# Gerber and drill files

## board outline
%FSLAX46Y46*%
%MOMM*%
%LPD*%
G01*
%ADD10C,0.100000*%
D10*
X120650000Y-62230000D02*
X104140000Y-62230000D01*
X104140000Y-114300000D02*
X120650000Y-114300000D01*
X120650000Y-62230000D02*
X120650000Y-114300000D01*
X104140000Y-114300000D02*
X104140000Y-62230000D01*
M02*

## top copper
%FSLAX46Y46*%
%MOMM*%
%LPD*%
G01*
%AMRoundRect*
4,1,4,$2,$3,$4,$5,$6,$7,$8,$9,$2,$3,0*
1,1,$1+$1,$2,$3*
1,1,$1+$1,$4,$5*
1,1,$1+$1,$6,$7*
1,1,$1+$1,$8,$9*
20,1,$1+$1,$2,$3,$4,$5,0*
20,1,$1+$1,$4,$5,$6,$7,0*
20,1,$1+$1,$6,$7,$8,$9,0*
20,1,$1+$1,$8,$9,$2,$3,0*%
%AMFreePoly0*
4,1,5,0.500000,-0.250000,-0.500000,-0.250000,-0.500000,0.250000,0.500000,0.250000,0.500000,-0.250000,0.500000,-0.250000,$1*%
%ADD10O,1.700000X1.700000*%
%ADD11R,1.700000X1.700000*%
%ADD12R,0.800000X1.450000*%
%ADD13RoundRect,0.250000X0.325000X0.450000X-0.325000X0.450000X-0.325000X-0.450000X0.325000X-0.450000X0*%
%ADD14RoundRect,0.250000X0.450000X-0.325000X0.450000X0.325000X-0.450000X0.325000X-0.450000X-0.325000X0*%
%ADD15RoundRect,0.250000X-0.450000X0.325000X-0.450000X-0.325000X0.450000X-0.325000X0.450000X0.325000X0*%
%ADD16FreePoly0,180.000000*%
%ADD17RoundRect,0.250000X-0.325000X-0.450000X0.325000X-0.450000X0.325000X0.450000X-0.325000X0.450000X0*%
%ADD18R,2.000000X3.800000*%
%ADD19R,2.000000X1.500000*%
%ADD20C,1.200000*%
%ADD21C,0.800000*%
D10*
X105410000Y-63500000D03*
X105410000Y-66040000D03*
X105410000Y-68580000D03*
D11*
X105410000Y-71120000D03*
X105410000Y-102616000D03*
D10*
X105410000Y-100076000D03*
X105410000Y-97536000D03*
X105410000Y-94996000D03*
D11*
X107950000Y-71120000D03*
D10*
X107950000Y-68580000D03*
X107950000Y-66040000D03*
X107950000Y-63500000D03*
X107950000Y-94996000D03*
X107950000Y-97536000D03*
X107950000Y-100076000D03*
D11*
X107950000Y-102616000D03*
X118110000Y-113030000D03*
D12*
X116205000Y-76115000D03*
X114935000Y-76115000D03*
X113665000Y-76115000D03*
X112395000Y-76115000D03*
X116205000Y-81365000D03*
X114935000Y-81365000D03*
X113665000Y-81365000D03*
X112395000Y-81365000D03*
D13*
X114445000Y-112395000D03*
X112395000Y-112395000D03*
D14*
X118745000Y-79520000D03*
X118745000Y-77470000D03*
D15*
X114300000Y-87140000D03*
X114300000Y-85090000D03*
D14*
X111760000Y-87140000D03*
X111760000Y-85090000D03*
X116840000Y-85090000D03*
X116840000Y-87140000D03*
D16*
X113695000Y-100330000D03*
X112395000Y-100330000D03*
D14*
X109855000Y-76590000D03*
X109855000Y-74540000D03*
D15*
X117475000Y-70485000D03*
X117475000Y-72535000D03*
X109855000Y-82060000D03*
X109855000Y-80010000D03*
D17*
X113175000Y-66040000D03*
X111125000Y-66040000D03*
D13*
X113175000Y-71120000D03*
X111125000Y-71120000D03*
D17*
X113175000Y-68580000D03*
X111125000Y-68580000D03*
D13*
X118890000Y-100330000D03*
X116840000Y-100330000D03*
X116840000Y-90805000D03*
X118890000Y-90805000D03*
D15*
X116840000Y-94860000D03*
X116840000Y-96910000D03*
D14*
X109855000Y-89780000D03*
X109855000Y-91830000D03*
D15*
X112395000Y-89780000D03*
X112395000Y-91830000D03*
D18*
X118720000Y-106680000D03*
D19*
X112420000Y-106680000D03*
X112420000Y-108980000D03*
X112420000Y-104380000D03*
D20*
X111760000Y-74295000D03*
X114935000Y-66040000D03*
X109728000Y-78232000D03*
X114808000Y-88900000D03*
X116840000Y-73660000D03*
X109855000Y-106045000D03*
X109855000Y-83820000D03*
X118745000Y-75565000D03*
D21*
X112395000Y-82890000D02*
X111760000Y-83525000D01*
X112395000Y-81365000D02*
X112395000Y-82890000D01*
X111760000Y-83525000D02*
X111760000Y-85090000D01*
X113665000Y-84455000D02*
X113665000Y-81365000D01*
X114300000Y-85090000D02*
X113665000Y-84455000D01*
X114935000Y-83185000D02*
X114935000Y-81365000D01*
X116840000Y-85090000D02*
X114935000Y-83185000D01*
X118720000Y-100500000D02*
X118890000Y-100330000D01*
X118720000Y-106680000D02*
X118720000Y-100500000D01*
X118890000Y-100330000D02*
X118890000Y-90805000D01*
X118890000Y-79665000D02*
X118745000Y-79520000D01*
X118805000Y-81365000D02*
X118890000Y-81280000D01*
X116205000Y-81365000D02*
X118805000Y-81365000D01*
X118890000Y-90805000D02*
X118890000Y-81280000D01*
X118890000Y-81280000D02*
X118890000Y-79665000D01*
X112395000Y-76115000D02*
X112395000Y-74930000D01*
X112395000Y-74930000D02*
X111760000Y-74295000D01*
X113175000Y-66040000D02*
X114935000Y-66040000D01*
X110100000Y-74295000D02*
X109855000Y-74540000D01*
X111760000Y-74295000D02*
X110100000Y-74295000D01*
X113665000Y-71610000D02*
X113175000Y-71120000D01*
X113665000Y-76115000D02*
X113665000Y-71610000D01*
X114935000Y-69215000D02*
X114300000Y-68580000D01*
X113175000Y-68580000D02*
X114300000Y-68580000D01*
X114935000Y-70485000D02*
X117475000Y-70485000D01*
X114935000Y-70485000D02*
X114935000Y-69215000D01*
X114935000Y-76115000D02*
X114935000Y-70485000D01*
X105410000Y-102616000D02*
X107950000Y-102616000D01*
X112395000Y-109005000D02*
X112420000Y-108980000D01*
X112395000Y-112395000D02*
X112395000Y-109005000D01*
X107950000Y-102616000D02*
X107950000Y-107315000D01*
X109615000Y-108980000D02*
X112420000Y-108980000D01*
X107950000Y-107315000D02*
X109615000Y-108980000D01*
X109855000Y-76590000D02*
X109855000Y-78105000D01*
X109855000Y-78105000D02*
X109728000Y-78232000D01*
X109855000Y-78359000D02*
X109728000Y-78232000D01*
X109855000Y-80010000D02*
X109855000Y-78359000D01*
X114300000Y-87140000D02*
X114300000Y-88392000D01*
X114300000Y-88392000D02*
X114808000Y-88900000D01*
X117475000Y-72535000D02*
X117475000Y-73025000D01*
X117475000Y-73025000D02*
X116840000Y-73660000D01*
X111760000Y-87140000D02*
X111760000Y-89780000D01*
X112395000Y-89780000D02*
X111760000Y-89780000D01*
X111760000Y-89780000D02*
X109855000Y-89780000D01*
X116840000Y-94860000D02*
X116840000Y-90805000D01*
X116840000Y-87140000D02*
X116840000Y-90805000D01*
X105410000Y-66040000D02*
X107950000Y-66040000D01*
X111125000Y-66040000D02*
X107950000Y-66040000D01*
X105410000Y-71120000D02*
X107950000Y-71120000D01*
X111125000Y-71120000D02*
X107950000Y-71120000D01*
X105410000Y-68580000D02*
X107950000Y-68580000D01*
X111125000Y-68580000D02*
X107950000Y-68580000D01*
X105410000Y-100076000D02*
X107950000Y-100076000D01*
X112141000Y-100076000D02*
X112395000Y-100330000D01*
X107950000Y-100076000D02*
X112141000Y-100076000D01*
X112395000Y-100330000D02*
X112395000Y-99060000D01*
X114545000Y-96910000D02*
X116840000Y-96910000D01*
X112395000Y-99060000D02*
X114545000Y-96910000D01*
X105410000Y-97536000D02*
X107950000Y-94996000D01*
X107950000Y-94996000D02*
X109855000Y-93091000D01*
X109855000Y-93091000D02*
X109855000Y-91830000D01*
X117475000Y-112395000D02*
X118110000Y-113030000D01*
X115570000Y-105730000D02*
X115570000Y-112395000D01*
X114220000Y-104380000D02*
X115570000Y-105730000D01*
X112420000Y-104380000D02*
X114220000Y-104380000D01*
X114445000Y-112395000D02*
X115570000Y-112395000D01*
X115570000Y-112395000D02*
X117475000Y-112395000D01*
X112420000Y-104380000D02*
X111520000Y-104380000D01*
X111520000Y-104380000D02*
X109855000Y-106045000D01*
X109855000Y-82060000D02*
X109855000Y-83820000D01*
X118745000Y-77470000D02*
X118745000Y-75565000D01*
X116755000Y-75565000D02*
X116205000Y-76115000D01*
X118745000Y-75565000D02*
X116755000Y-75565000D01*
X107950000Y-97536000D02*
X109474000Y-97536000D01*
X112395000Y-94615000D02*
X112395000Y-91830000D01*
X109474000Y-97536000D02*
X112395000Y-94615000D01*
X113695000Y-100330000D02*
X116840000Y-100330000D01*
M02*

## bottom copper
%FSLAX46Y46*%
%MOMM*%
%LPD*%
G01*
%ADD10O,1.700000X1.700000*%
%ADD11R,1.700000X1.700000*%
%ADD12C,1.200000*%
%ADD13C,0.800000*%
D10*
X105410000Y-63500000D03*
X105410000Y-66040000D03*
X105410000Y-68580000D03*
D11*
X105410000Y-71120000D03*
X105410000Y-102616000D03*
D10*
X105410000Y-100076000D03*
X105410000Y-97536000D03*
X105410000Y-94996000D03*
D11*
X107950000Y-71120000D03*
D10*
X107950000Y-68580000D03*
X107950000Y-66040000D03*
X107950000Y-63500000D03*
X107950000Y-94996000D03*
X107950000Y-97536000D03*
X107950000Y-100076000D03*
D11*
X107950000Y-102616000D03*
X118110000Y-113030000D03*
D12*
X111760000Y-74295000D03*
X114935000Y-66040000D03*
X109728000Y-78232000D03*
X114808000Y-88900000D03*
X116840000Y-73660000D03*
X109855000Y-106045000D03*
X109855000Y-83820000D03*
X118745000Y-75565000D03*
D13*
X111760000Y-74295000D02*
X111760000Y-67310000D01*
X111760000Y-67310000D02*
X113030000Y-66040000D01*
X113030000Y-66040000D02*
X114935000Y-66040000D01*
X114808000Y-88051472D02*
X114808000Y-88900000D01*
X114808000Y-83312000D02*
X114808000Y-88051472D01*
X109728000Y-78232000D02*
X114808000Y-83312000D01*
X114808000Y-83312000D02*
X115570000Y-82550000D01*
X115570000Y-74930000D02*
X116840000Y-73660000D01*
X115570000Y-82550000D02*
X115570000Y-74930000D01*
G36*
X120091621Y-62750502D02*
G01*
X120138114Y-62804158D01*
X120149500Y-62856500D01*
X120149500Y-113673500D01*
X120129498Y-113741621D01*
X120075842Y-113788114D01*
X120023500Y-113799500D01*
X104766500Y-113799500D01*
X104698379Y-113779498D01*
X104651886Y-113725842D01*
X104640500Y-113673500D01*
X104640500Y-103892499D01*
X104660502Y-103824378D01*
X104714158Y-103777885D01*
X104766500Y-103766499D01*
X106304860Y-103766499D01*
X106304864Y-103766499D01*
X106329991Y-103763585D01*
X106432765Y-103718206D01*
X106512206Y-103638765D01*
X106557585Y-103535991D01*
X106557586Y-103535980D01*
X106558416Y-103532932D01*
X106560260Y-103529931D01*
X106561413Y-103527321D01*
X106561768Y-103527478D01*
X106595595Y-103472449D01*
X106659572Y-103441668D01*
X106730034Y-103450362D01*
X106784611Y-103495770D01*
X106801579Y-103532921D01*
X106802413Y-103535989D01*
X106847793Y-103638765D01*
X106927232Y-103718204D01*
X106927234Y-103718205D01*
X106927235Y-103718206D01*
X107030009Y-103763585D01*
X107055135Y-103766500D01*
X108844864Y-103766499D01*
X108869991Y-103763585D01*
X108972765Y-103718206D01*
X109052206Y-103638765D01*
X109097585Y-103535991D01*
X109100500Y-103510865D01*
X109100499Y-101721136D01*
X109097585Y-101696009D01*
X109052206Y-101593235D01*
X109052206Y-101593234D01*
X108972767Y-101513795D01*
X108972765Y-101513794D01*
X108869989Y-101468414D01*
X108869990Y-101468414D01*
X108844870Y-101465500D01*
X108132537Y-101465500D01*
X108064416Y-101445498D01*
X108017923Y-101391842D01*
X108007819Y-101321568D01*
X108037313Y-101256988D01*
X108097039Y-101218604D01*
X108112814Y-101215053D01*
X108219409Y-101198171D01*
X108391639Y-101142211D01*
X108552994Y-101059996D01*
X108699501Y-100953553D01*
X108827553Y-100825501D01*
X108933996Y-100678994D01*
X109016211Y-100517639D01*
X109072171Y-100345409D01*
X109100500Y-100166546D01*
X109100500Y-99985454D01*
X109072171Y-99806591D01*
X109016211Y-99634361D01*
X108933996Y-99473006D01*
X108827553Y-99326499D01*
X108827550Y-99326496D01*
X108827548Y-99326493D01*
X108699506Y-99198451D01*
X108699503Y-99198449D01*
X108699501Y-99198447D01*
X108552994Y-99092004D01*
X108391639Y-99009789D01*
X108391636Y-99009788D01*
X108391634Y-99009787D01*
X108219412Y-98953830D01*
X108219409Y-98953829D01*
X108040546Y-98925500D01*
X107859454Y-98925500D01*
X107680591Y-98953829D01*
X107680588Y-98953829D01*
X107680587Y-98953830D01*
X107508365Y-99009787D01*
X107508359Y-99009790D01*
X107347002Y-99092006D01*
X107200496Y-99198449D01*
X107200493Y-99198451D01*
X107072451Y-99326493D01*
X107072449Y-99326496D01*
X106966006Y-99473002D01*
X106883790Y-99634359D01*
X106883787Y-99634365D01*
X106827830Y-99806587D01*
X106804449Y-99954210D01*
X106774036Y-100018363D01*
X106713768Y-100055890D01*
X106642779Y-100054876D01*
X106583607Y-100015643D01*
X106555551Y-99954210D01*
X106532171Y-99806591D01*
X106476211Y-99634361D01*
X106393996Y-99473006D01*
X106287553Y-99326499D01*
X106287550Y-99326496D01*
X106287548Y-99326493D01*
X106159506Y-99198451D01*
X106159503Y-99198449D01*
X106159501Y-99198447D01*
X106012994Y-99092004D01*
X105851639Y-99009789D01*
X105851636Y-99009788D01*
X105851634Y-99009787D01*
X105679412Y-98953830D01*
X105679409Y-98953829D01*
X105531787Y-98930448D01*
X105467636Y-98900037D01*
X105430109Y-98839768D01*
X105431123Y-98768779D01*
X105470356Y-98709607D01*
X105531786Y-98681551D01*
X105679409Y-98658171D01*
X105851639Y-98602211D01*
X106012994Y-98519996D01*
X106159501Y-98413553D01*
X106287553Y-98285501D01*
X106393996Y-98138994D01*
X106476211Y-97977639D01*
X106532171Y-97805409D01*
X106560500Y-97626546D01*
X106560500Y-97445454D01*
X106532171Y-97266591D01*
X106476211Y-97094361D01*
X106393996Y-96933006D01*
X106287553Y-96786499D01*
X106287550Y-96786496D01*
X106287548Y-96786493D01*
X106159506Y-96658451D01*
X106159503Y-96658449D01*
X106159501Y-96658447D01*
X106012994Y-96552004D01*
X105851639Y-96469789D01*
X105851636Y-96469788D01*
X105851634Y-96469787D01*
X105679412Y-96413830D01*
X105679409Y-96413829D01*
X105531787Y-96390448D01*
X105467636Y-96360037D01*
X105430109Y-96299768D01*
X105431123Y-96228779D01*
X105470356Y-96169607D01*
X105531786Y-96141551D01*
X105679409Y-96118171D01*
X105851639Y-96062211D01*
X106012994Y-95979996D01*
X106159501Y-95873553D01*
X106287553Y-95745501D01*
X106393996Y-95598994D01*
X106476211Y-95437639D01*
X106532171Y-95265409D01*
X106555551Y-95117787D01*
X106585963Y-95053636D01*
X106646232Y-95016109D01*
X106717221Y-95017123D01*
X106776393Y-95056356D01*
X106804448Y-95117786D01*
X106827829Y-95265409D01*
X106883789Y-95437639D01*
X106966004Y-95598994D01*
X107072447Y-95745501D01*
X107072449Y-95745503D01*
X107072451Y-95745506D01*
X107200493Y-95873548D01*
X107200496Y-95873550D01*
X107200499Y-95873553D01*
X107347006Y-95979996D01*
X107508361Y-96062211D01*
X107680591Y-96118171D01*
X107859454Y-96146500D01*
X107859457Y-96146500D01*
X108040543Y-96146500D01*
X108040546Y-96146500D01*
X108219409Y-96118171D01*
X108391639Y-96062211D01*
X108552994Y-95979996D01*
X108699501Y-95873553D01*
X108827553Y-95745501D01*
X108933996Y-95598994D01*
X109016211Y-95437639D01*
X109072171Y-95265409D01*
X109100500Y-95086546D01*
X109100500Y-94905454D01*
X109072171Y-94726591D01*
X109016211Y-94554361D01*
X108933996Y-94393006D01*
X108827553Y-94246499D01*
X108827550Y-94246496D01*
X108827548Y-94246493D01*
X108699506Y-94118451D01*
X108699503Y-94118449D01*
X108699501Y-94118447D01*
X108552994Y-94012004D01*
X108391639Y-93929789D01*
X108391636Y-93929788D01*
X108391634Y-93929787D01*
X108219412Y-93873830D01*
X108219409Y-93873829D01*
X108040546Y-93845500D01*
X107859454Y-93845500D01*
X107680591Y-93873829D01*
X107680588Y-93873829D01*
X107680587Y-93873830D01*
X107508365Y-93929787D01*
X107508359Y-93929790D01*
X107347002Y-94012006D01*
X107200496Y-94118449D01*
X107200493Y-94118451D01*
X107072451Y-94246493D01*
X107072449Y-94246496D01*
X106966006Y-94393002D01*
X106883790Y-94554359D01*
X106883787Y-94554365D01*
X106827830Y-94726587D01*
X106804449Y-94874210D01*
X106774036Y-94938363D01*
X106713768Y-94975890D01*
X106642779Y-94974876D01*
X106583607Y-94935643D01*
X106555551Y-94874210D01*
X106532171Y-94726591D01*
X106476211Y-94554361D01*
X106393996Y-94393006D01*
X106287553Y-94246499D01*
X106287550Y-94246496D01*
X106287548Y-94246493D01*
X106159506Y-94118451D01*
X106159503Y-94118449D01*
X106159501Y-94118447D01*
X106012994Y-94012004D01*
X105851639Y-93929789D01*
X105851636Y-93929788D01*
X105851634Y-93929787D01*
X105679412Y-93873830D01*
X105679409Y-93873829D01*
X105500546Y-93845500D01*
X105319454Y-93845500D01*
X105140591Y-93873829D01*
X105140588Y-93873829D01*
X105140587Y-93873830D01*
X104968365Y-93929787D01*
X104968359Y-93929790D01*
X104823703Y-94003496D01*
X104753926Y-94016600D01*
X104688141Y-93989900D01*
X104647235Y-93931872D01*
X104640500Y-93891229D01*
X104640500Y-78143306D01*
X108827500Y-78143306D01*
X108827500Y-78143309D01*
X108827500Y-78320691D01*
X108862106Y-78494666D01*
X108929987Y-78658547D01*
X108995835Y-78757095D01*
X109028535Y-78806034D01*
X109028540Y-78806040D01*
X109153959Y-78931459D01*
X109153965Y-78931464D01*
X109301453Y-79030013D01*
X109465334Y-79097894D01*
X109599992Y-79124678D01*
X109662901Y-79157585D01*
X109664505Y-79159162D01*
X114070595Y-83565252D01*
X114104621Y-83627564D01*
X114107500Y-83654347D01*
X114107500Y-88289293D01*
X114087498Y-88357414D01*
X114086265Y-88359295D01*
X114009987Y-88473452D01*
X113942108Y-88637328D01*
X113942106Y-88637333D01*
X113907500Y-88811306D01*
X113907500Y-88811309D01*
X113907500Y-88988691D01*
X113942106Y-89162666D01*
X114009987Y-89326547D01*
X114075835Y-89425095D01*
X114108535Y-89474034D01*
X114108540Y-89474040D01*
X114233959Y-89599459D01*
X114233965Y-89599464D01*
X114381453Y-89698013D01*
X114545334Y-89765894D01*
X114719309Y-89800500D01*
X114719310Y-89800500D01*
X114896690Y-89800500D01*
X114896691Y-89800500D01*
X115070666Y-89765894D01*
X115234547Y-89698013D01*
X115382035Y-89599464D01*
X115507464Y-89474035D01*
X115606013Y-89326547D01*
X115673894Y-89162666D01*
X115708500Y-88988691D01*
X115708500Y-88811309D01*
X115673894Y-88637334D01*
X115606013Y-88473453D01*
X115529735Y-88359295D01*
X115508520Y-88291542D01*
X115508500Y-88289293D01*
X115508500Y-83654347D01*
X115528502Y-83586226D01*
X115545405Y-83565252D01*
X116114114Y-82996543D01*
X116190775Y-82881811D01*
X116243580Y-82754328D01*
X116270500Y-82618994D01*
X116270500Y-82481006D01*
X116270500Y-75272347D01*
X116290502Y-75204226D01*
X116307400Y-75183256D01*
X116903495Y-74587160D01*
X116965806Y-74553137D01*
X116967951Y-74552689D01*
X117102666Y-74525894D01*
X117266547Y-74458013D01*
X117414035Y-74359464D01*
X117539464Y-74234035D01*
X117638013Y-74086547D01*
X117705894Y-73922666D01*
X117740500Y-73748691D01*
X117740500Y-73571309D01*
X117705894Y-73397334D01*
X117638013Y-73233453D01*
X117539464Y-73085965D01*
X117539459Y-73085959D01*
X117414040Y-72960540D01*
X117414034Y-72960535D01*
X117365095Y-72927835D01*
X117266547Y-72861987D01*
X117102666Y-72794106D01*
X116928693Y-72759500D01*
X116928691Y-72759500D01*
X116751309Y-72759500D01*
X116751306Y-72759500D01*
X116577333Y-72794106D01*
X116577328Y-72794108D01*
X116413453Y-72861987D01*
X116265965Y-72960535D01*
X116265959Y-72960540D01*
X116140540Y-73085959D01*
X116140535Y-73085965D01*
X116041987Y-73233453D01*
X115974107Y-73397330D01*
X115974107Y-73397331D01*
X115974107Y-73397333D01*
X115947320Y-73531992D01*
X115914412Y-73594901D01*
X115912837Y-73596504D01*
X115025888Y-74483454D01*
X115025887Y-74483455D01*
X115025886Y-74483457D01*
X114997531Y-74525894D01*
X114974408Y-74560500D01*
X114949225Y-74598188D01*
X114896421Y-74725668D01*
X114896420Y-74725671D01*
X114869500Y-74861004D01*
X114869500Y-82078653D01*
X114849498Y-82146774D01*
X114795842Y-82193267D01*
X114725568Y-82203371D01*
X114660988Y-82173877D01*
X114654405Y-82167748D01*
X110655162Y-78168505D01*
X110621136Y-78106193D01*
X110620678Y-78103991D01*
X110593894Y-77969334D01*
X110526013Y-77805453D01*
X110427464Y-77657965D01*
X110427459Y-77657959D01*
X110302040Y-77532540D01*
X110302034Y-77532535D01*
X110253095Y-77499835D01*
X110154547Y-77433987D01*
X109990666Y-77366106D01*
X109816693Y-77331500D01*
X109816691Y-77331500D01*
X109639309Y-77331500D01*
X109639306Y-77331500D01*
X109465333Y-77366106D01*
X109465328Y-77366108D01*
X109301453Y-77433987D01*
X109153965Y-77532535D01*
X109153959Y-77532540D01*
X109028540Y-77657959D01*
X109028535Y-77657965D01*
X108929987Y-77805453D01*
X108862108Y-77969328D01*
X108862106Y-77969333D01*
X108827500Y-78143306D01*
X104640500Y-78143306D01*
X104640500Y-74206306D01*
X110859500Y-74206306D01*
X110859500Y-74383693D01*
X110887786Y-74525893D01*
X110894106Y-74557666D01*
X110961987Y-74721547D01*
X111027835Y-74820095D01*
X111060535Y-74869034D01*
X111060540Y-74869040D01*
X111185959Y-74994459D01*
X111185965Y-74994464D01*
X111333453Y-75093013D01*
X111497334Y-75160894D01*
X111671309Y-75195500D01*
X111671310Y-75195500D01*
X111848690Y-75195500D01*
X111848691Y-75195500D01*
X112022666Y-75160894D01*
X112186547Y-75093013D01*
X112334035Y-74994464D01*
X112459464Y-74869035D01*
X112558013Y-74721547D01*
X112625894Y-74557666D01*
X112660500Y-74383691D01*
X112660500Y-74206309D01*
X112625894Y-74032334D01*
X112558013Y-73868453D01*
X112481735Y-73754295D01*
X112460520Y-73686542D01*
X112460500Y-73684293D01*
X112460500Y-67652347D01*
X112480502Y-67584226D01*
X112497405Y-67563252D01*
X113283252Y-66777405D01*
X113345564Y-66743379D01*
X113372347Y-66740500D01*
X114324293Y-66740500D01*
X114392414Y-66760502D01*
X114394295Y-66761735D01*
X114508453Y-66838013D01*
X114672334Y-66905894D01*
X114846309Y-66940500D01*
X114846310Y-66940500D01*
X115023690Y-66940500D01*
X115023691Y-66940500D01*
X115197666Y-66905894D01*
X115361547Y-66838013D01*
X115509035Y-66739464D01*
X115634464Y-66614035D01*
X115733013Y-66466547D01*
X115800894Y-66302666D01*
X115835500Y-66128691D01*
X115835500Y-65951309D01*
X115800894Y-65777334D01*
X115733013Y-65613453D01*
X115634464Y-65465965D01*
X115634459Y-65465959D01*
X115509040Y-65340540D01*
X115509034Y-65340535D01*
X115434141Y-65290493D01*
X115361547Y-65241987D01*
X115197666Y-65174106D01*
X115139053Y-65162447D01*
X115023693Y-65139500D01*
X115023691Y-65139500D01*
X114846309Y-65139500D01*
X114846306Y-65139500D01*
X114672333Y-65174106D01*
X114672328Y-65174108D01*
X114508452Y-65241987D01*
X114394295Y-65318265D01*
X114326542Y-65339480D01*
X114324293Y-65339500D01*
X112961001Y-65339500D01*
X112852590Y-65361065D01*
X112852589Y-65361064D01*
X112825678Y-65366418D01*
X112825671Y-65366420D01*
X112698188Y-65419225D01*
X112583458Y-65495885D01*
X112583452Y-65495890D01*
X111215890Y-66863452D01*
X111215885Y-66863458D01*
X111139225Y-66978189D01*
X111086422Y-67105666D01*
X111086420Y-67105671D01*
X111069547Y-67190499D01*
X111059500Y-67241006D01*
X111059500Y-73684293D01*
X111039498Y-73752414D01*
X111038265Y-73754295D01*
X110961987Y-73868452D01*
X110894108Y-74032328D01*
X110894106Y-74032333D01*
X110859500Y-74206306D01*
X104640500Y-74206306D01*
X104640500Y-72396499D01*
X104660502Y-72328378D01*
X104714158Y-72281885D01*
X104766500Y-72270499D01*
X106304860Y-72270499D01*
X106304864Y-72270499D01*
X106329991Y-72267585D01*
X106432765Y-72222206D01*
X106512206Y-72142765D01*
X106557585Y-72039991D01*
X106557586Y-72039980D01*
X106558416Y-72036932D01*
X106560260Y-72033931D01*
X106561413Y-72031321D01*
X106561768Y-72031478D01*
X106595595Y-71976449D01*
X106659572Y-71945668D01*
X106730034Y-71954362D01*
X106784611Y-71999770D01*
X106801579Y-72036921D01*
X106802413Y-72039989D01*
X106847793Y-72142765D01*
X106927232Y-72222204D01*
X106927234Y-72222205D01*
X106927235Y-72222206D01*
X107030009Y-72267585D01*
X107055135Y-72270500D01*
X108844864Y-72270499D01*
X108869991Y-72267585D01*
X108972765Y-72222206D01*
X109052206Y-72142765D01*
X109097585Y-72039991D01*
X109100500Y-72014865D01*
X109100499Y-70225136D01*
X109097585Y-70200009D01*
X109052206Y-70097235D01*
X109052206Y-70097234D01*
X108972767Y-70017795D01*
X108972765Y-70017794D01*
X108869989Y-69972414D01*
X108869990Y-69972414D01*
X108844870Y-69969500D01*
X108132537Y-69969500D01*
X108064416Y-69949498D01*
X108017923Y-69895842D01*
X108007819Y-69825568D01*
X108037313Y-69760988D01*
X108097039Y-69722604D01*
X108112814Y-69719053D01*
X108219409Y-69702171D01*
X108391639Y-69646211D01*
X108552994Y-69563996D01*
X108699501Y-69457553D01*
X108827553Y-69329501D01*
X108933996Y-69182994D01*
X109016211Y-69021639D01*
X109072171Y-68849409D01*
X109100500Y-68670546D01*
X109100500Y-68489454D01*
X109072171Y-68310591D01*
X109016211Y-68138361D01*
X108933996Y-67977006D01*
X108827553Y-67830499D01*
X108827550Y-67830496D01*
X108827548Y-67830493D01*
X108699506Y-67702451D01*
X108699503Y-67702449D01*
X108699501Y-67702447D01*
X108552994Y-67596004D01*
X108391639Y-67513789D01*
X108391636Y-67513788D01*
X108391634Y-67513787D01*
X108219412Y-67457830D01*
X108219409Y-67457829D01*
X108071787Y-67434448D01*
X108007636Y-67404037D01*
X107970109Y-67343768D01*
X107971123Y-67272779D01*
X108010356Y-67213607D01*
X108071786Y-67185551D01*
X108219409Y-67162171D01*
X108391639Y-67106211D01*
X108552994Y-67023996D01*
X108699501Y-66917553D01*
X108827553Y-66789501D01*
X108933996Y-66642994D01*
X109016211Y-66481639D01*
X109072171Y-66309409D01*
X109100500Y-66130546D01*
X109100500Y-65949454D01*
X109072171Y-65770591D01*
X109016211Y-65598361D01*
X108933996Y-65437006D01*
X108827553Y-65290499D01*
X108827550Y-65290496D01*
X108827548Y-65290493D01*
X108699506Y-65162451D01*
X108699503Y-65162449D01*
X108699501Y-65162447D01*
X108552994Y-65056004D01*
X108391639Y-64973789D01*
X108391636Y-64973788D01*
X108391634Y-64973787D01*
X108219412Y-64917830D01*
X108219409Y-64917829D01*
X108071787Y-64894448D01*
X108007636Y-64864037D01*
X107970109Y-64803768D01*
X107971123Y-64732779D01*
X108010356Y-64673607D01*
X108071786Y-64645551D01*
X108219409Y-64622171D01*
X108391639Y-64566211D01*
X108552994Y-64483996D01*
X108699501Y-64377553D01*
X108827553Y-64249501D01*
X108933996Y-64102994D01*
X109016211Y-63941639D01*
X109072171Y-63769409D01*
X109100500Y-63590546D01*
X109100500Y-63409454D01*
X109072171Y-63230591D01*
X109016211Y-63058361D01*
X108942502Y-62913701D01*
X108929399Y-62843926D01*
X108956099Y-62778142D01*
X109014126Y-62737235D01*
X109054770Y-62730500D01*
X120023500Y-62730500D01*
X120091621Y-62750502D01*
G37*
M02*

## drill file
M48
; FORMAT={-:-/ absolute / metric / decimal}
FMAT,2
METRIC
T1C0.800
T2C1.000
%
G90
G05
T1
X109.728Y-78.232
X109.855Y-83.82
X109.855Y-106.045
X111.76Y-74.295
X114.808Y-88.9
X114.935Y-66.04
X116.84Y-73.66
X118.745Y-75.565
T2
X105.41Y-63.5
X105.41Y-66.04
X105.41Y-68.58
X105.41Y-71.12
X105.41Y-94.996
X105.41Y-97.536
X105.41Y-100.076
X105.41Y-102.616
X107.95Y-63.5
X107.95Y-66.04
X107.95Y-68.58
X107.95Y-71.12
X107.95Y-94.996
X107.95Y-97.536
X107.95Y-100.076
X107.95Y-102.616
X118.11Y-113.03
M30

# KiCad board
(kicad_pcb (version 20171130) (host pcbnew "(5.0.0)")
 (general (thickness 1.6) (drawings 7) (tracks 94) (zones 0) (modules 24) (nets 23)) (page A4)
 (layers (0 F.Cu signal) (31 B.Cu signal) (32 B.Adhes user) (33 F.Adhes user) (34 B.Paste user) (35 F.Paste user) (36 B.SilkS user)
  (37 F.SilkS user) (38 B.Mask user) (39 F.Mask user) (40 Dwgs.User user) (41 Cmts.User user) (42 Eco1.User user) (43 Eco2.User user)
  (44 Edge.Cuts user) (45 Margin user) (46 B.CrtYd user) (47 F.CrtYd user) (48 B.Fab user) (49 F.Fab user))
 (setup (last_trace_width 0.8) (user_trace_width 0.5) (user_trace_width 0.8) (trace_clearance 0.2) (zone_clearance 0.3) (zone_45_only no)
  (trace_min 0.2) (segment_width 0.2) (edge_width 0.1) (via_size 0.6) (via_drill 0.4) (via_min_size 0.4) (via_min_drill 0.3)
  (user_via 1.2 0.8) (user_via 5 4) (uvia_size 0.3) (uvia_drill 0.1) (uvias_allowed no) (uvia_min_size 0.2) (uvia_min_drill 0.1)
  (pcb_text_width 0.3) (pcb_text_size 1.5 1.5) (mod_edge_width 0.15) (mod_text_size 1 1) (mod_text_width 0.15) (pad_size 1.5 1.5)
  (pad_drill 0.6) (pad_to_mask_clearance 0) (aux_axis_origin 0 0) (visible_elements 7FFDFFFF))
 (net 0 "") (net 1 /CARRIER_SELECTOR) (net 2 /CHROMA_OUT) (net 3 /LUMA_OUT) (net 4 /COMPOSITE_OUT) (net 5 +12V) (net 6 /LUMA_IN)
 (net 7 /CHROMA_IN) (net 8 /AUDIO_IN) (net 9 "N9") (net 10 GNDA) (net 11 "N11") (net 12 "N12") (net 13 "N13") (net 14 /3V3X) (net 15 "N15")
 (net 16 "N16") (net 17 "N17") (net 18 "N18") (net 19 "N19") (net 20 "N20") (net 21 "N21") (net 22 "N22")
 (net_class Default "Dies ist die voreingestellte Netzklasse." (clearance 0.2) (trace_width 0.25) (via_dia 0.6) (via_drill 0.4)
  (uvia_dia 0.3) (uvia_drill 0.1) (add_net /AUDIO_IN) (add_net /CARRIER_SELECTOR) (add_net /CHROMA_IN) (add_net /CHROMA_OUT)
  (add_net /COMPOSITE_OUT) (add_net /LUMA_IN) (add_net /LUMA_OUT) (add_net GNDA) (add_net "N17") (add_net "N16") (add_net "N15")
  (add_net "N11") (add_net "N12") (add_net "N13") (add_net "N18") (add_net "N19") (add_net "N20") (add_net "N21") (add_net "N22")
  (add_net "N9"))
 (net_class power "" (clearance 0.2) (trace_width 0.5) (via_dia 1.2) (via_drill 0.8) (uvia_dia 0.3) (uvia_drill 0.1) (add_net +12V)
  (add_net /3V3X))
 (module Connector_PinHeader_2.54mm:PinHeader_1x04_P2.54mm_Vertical (layer F.Cu) (at 105.41 71.12 180)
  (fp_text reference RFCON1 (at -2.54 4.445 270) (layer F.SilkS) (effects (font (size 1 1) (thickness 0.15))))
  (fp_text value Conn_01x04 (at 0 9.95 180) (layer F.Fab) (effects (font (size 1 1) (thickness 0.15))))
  (pad 4 thru_hole oval (at 0 7.62 180) (size 1.7 1.7) (drill 1) (layers *.Cu *.Mask) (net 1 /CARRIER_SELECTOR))
  (pad 3 thru_hole oval (at 0 5.08 180) (size 1.7 1.7) (drill 1) (layers *.Cu *.Mask) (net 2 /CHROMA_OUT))
  (pad 2 thru_hole oval (at 0 2.54 180) (size 1.7 1.7) (drill 1) (layers *.Cu *.Mask) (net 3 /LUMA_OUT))
  (pad 1 thru_hole rect (at 0 0 180) (size 1.7 1.7) (drill 1) (layers *.Cu *.Mask) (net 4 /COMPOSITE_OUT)))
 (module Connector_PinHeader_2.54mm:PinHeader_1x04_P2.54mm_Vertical (layer F.Cu) (at 105.41 102.616 180)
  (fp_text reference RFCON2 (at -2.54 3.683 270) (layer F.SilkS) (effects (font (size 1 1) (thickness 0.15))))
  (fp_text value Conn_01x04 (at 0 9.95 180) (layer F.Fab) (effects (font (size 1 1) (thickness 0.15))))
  (pad 1 thru_hole rect (at 0 0 180) (size 1.7 1.7) (drill 1) (layers *.Cu *.Mask) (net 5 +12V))
  (pad 2 thru_hole oval (at 0 2.54 180) (size 1.7 1.7) (drill 1) (layers *.Cu *.Mask) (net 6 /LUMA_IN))
  (pad 3 thru_hole oval (at 0 5.08 180) (size 1.7 1.7) (drill 1) (layers *.Cu *.Mask) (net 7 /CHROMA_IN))
  (pad 4 thru_hole oval (at 0 7.62 180) (size 1.7 1.7) (drill 1) (layers *.Cu *.Mask) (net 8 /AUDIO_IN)))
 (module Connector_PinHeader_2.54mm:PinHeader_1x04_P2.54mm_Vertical (layer F.Cu) (at 107.95 71.12 180)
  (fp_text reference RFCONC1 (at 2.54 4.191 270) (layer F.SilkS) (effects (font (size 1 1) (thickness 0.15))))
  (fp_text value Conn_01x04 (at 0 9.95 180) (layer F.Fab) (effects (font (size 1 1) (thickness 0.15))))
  (pad 1 thru_hole rect (at 0 0 180) (size 1.7 1.7) (drill 1) (layers *.Cu *.Mask) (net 4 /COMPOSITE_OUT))
  (pad 2 thru_hole oval (at 0 2.54 180) (size 1.7 1.7) (drill 1) (layers *.Cu *.Mask) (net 3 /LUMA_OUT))
  (pad 3 thru_hole oval (at 0 5.08 180) (size 1.7 1.7) (drill 1) (layers *.Cu *.Mask) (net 2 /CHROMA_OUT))
  (pad 4 thru_hole oval (at 0 7.62 180) (size 1.7 1.7) (drill 1) (layers *.Cu *.Mask) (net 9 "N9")))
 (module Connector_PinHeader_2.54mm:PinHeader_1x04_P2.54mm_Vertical (layer F.Cu) (at 107.95 102.616 180)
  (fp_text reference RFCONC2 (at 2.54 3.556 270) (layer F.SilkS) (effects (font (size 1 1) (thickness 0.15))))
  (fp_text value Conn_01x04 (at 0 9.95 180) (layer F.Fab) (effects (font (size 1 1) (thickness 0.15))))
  (pad 4 thru_hole oval (at 0 7.62 180) (size 1.7 1.7) (drill 1) (layers *.Cu *.Mask) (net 7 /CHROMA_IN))
  (pad 3 thru_hole oval (at 0 5.08 180) (size 1.7 1.7) (drill 1) (layers *.Cu *.Mask) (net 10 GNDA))
  (pad 2 thru_hole oval (at 0 2.54 180) (size 1.7 1.7) (drill 1) (layers *.Cu *.Mask) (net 6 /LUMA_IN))
  (pad 1 thru_hole rect (at 0 0 180) (size 1.7 1.7) (drill 1) (layers *.Cu *.Mask) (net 5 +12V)))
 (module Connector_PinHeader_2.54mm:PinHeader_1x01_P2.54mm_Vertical (layer F.Cu) (at 118.11 113.03)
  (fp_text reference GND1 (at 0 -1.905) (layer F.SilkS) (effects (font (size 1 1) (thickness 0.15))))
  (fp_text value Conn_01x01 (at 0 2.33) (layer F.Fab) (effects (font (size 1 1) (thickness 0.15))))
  (pad 1 thru_hole rect (at 0 0) (size 1.7 1.7) (drill 1) (layers *.Cu *.Mask) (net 10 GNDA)))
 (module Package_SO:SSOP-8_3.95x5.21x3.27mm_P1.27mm (layer F.Cu) (at 114.3 78.74 90)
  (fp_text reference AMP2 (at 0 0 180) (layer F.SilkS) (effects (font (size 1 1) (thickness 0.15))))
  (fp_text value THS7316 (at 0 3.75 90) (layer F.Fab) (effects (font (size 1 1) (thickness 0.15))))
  (pad 5 smd rect (at 2.625 1.905 90) (size 1.45 0.8) (layers F.Cu F.Paste F.Mask) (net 10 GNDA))
  (pad 6 smd rect (at 2.625 0.635 90) (size 1.45 0.8) (layers F.Cu F.Paste F.Mask) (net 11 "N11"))
  (pad 7 smd rect (at 2.625 -0.635 90) (size 1.45 0.8) (layers F.Cu F.Paste F.Mask) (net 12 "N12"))
  (pad 8 smd rect (at 2.625 -1.905 90) (size 1.45 0.8) (layers F.Cu F.Paste F.Mask) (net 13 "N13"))
  (pad 4 smd rect (at -2.625 1.905 90) (size 1.45 0.8) (layers F.Cu F.Paste F.Mask) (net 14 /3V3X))
  (pad 3 smd rect (at -2.625 0.635 90) (size 1.45 0.8) (layers F.Cu F.Paste F.Mask) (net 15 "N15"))
  (pad 2 smd rect (at -2.625 -0.635 90) (size 1.45 0.8) (layers F.Cu F.Paste F.Mask) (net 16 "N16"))
  (pad 1 smd rect (at -2.625 -1.905 90) (size 1.45 0.8) (layers F.Cu F.Paste F.Mask) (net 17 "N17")))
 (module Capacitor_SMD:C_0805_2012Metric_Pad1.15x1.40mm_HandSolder (layer F.Cu) (at 113.42 112.395 180)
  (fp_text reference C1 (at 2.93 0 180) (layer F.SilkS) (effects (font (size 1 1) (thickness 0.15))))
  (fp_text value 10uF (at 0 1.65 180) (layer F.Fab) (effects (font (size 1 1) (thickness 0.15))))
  (pad 1 smd roundrect (at -1.025 0 180) (size 1.15 1.4) (layers F.Cu F.Paste F.Mask) (roundrect_rratio 0.217391) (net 10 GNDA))
  (pad 2 smd roundrect (at 1.025 0 180) (size 1.15 1.4) (layers F.Cu F.Paste F.Mask) (roundrect_rratio 0.217391) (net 5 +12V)))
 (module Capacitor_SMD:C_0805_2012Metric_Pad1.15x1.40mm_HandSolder (layer F.Cu) (at 118.745 78.495 90)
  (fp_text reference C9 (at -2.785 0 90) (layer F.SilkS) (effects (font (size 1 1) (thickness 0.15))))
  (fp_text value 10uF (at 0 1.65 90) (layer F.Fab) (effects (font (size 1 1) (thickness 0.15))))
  (pad 1 smd roundrect (at -1.025 0 90) (size 1.15 1.4) (layers F.Cu F.Paste F.Mask) (roundrect_rratio 0.217391) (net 14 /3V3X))
  (pad 2 smd roundrect (at 1.025 0 90) (size 1.15 1.4) (layers F.Cu F.Paste F.Mask) (roundrect_rratio 0.217391) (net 10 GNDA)))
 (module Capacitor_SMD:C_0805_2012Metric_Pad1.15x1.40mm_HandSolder (layer F.Cu) (at 114.3 86.115 270)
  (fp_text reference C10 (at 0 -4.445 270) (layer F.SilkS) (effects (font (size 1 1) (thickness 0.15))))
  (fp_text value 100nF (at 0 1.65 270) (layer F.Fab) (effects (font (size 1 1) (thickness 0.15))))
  (pad 2 smd roundrect (at 1.025 0 270) (size 1.15 1.4) (layers F.Cu F.Paste F.Mask) (roundrect_rratio 0.217391) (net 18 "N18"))
  (pad 1 smd roundrect (at -1.025 0 270) (size 1.15 1.4) (layers F.Cu F.Paste F.Mask) (roundrect_rratio 0.217391) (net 16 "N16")))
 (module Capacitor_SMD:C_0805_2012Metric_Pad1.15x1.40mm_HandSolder (layer F.Cu) (at 111.76 86.115 90)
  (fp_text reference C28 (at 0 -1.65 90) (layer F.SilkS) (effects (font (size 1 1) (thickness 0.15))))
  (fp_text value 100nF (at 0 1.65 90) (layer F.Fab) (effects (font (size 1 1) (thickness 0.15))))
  (pad 1 smd roundrect (at -1.025 0 90) (size 1.15 1.4) (layers F.Cu F.Paste F.Mask) (roundrect_rratio 0.217391) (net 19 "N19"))
  (pad 2 smd roundrect (at 1.025 0 90) (size 1.15 1.4) (layers F.Cu F.Paste F.Mask) (roundrect_rratio 0.217391) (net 17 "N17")))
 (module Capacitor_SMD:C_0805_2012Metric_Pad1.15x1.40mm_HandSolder (layer F.Cu) (at 116.84 86.115 90)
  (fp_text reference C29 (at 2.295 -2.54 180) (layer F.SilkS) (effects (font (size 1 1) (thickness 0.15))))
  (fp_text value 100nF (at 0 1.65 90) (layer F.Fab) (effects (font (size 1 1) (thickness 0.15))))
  (pad 2 smd roundrect (at 1.025 0 90) (size 1.15 1.4) (layers F.Cu F.Paste F.Mask) (roundrect_rratio 0.217391) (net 15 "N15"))
  (pad 1 smd roundrect (at -1.025 0 90) (size 1.15 1.4) (layers F.Cu F.Paste F.Mask) (roundrect_rratio 0.217391) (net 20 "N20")))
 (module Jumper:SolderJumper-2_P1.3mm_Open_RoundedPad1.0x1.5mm (layer F.Cu) (at 113.045 100.33 180)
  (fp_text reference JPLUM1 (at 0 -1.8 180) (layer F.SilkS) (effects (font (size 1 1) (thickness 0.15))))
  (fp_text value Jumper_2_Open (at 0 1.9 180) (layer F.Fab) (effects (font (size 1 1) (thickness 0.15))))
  (pad 1 smd custom (at -0.65 0 180) (size 1 0.5) (layers F.Cu F.Mask) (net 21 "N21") (zone_connect 0)
   (options (clearance outline) (anchor rect)) (primitives))
  (pad 2 smd custom (at 0.65 0 180) (size 1 0.5) (layers F.Cu F.Mask) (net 6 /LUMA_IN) (zone_connect 0)
   (options (clearance outline) (anchor rect)) (primitives)))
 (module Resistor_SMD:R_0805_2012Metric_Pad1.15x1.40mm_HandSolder (layer F.Cu) (at 109.855 75.565 90)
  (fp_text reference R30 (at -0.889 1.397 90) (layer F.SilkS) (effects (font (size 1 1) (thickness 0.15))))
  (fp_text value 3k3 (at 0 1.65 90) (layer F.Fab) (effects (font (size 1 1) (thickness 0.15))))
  (pad 1 smd roundrect (at -1.025 0 90) (size 1.15 1.4) (layers F.Cu F.Paste F.Mask) (roundrect_rratio 0.217391) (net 18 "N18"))
  (pad 2 smd roundrect (at 1.025 0 90) (size 1.15 1.4) (layers F.Cu F.Paste F.Mask) (roundrect_rratio 0.217391) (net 13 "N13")))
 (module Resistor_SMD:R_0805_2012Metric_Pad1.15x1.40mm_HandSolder (layer F.Cu) (at 117.475 71.51 270)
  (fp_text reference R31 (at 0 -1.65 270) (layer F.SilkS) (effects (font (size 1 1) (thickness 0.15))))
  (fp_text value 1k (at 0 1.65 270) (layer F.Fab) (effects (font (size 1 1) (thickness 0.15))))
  (pad 1 smd roundrect (at -1.025 0 270) (size 1.15 1.4) (layers F.Cu F.Paste F.Mask) (roundrect_rratio 0.217391) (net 11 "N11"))
  (pad 2 smd roundrect (at 1.025 0 270) (size 1.15 1.4) (layers F.Cu F.Paste F.Mask) (roundrect_rratio 0.217391) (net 18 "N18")))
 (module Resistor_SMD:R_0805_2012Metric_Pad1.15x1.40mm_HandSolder (layer F.Cu) (at 109.855 81.035 270)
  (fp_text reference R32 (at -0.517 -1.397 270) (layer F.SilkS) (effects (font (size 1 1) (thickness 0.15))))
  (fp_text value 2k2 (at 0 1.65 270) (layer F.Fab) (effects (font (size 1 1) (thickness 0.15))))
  (pad 2 smd roundrect (at 1.025 0 270) (size 1.15 1.4) (layers F.Cu F.Paste F.Mask) (roundrect_rratio 0.217391) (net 10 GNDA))
  (pad 1 smd roundrect (at -1.025 0 270) (size 1.15 1.4) (layers F.Cu F.Paste F.Mask) (roundrect_rratio 0.217391) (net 18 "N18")))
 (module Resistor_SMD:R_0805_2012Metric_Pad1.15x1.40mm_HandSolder (layer F.Cu) (at 112.15 66.04)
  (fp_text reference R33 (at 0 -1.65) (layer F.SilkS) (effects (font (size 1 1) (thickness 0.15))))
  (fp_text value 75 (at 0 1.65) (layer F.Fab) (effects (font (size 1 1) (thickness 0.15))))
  (pad 2 smd roundrect (at 1.025 0) (size 1.15 1.4) (layers F.Cu F.Paste F.Mask) (roundrect_rratio 0.217391) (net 13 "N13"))
  (pad 1 smd roundrect (at -1.025 0) (size 1.15 1.4) (layers F.Cu F.Paste F.Mask) (roundrect_rratio 0.217391) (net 2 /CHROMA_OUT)))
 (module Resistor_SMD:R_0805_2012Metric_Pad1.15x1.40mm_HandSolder (layer F.Cu) (at 112.15 71.12 180)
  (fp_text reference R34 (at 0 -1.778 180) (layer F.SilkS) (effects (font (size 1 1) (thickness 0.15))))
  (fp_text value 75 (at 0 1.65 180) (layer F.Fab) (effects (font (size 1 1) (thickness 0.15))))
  (pad 1 smd roundrect (at -1.025 0 180) (size 1.15 1.4) (layers F.Cu F.Paste F.Mask) (roundrect_rratio 0.217391) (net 12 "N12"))
  (pad 2 smd roundrect (at 1.025 0 180) (size 1.15 1.4) (layers F.Cu F.Paste F.Mask) (roundrect_rratio 0.217391) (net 4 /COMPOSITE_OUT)))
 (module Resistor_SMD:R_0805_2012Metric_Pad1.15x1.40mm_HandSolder (layer F.Cu) (at 112.15 68.58)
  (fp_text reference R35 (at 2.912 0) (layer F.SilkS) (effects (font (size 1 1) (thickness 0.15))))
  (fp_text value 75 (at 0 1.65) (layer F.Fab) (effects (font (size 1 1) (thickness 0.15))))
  (pad 2 smd roundrect (at 1.025 0) (size 1.15 1.4) (layers F.Cu F.Paste F.Mask) (roundrect_rratio 0.217391) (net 11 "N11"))
  (pad 1 smd roundrect (at -1.025 0) (size 1.15 1.4) (layers F.Cu F.Paste F.Mask) (roundrect_rratio 0.217391) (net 3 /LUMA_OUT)))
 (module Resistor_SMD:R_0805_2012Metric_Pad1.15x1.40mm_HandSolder (layer F.Cu) (at 117.865 100.33 180)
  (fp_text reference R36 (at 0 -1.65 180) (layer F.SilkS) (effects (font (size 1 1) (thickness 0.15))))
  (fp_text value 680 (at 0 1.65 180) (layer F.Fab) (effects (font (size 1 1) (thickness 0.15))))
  (pad 1 smd roundrect (at -1.025 0 180) (size 1.15 1.4) (layers F.Cu F.Paste F.Mask) (roundrect_rratio 0.217391) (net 14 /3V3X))
  (pad 2 smd roundrect (at 1.025 0 180) (size 1.15 1.4) (layers F.Cu F.Paste F.Mask) (roundrect_rratio 0.217391) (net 21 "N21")))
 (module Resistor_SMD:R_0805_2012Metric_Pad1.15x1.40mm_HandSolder (layer F.Cu) (at 117.865 90.805 180)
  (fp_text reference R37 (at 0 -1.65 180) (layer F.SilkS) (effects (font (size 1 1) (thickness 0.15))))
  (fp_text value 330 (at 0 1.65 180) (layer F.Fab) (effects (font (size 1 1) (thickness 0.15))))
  (pad 2 smd roundrect (at 1.025 0 180) (size 1.15 1.4) (layers F.Cu F.Paste F.Mask) (roundrect_rratio 0.217391) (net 20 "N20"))
  (pad 1 smd roundrect (at -1.025 0 180) (size 1.15 1.4) (layers F.Cu F.Paste F.Mask) (roundrect_rratio 0.217391) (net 14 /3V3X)))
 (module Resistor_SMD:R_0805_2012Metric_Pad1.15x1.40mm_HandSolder (layer F.Cu) (at 116.84 95.885 270)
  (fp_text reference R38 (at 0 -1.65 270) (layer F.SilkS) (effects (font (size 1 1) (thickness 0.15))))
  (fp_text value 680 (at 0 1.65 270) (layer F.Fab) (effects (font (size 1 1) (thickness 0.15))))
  (pad 1 smd roundrect (at -1.025 0 270) (size 1.15 1.4) (layers F.Cu F.Paste F.Mask) (roundrect_rratio 0.217391) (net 20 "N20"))
  (pad 2 smd roundrect (at 1.025 0 270) (size 1.15 1.4) (layers F.Cu F.Paste F.Mask) (roundrect_rratio 0.217391) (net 6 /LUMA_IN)))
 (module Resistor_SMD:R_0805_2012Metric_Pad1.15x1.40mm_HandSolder (layer F.Cu) (at 109.855 90.805 90)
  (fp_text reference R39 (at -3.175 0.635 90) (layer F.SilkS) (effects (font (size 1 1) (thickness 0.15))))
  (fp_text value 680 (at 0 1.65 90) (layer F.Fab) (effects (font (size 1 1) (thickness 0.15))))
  (pad 2 smd roundrect (at 1.025 0 90) (size 1.15 1.4) (layers F.Cu F.Paste F.Mask) (roundrect_rratio 0.217391) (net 19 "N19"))
  (pad 1 smd roundrect (at -1.025 0 90) (size 1.15 1.4) (layers F.Cu F.Paste F.Mask) (roundrect_rratio 0.217391) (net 7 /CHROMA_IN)))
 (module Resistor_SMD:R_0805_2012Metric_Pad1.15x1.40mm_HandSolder (layer F.Cu) (at 112.395 90.805 270)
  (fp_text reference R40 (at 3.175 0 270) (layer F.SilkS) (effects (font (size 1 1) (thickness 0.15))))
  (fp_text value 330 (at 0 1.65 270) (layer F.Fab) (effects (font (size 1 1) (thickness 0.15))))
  (pad 1 smd roundrect (at -1.025 0 270) (size 1.15 1.4) (layers F.Cu F.Paste F.Mask) (roundrect_rratio 0.217391) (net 19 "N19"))
  (pad 2 smd roundrect (at 1.025 0 270) (size 1.15 1.4) (layers F.Cu F.Paste F.Mask) (roundrect_rratio 0.217391) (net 10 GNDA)))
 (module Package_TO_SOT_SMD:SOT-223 (layer F.Cu) (at 115.57 106.68)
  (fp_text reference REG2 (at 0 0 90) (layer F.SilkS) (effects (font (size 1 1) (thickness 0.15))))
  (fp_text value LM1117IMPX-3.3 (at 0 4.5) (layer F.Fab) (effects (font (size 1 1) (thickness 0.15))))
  (pad 4 smd rect (at 3.15 0) (size 2 3.8) (layers F.Cu F.Paste F.Mask) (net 14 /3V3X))
  (pad 2 smd rect (at -3.15 0) (size 2 1.5) (layers F.Cu F.Paste F.Mask) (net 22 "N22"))
  (pad 3 smd rect (at -3.15 2.3) (size 2 1.5) (layers F.Cu F.Paste F.Mask) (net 5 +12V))
  (pad 1 smd rect (at -3.15 -2.3) (size 2 1.5) (layers F.Cu F.Paste F.Mask) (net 10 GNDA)))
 (gr_line (start 120.65 62.23) (end 104.14 62.23) (layer Edge.Cuts) (width 0.1))
 (gr_line (start 104.14 114.3) (end 120.65 114.3) (layer Edge.Cuts) (width 0.1))
 (gr_line (start 120.65 62.23) (end 120.65 114.3) (layer Edge.Cuts) (width 0.1))
 (gr_line (start 104.14 114.3) (end 104.14 62.23) (layer Edge.Cuts) (width 0.1))
 (segment (start 112.395 82.89) (end 111.76 83.525) (width 0.8) (layer F.Cu) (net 17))
 (segment (start 112.395 81.365) (end 112.395 82.89) (width 0.8) (layer F.Cu) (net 17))
 (segment (start 111.76 83.525) (end 111.76 85.09) (width 0.8) (layer F.Cu) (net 17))
 (segment (start 113.665 84.455) (end 113.665 81.365) (width 0.8) (layer F.Cu) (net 16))
 (segment (start 114.3 85.09) (end 113.665 84.455) (width 0.8) (layer F.Cu) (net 16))
 (segment (start 114.935 83.185) (end 114.935 81.365) (width 0.8) (layer F.Cu) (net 15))
 (segment (start 116.84 85.09) (end 114.935 83.185) (width 0.8) (layer F.Cu) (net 15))
 (segment (start 118.72 100.5) (end 118.89 100.33) (width 0.8) (layer F.Cu) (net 14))
 (segment (start 118.72 106.68) (end 118.72 100.5) (width 0.8) (layer F.Cu) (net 14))
 (segment (start 118.89 100.33) (end 118.89 90.805) (width 0.8) (layer F.Cu) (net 14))
 (segment (start 118.89 79.665) (end 118.745 79.52) (width 0.8) (layer F.Cu) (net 14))
 (segment (start 118.805 81.365) (end 118.89 81.28) (width 0.8) (layer F.Cu) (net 14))
 (segment (start 116.205 81.365) (end 118.805 81.365) (width 0.8) (layer F.Cu) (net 14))
 (segment (start 118.89 90.805) (end 118.89 81.28) (width 0.8) (layer F.Cu) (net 14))
 (segment (start 118.89 81.28) (end 118.89 79.665) (width 0.8) (layer F.Cu) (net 14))
 (via (at 111.76 74.295) (size 1.2) (drill 0.8) (layers F.Cu B.Cu) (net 13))
 (segment (start 112.395 76.115) (end 112.395 74.93) (width 0.8) (layer F.Cu) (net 13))
 (segment (start 112.395 74.93) (end 111.76 74.295) (width 0.8) (layer F.Cu) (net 13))
 (segment (start 111.76 74.295) (end 111.76 67.31) (width 0.8) (layer B.Cu) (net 13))
 (segment (start 111.76 67.31) (end 113.03 66.04) (width 0.8) (layer B.Cu) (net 13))
 (via (at 114.935 66.04) (size 1.2) (drill 0.8) (layers F.Cu B.Cu) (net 13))
 (segment (start 113.03 66.04) (end 114.935 66.04) (width 0.8) (layer B.Cu) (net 13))
 (segment (start 113.175 66.04) (end 114.935 66.04) (width 0.8) (layer F.Cu) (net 13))
 (segment (start 110.1 74.295) (end 109.855 74.54) (width 0.8) (layer F.Cu) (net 13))
 (segment (start 111.76 74.295) (end 110.1 74.295) (width 0.8) (layer F.Cu) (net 13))
 (segment (start 113.665 71.61) (end 113.175 71.12) (width 0.8) (layer F.Cu) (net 12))
 (segment (start 113.665 76.115) (end 113.665 71.61) (width 0.8) (layer F.Cu) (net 12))
 (segment (start 114.935 69.215) (end 114.3 68.58) (width 0.8) (layer F.Cu) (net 11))
 (segment (start 113.175 68.58) (end 114.3 68.58) (width 0.8) (layer F.Cu) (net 11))
 (segment (start 114.935 70.485) (end 117.475 70.485) (width 0.8) (layer F.Cu) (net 11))
 (segment (start 114.935 70.485) (end 114.935 69.215) (width 0.8) (layer F.Cu) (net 11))
 (segment (start 114.935 76.115) (end 114.935 70.485) (width 0.8) (layer F.Cu) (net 11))
 (segment (start 105.41 102.616) (end 107.95 102.616) (width 0.8) (layer F.Cu) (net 5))
 (segment (start 112.395 109.005) (end 112.42 108.98) (width 0.8) (layer F.Cu) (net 5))
 (segment (start 112.395 112.395) (end 112.395 109.005) (width 0.8) (layer F.Cu) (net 5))
 (segment (start 107.95 102.616) (end 107.95 107.315) (width 0.8) (layer F.Cu) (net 5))
 (segment (start 109.615 108.98) (end 112.42 108.98) (width 0.8) (layer F.Cu) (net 5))
 (segment (start 107.95 107.315) (end 109.615 108.98) (width 0.8) (layer F.Cu) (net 5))
 (via (at 109.728 78.232) (size 1.2) (drill 0.8) (layers F.Cu B.Cu) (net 18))
 (segment (start 109.855 76.59) (end 109.855 78.105) (width 0.8) (layer F.Cu) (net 18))
 (segment (start 109.855 78.105) (end 109.728 78.232) (width 0.8) (layer F.Cu) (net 18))
 (segment (start 109.855 78.359) (end 109.728 78.232) (width 0.8) (layer F.Cu) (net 18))
 (segment (start 109.855 80.01) (end 109.855 78.359) (width 0.8) (layer F.Cu) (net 18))
 (segment (start 114.3 87.14) (end 114.3 88.392) (width 0.8) (layer F.Cu) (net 18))
 (segment (start 114.3 88.392) (end 114.808 88.9) (width 0.8) (layer F.Cu) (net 18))
 (segment (start 114.808 88.051472) (end 114.808 88.9) (width 0.8) (layer B.Cu) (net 18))
 (segment (start 114.808 83.312) (end 114.808 88.051472) (width 0.8) (layer B.Cu) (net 18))
 (via (at 114.808 88.9) (size 1.2) (drill 0.8) (layers F.Cu B.Cu) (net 18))
 (via (at 116.84 73.66) (size 1.2) (drill 0.8) (layers F.Cu B.Cu) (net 18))
 (segment (start 117.475 72.535) (end 117.475 73.025) (width 0.8) (layer F.Cu) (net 18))
 (segment (start 117.475 73.025) (end 116.84 73.66) (width 0.8) (layer F.Cu) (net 18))
 (segment (start 109.728 78.232) (end 114.808 83.312) (width 0.8) (layer B.Cu) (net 18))
 (segment (start 114.808 83.312) (end 115.57 82.55) (width 0.8) (layer B.Cu) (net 18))
 (segment (start 115.57 74.93) (end 116.84 73.66) (width 0.8) (layer B.Cu) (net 18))
 (segment (start 115.57 82.55) (end 115.57 74.93) (width 0.8) (layer B.Cu) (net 18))
 (segment (start 111.76 87.14) (end 111.76 89.78) (width 0.8) (layer F.Cu) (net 19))
 (segment (start 112.395 89.78) (end 111.76 89.78) (width 0.8) (layer F.Cu) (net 19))
 (segment (start 111.76 89.78) (end 109.855 89.78) (width 0.8) (layer F.Cu) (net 19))
 (segment (start 116.84 94.86) (end 116.84 90.805) (width 0.8) (layer F.Cu) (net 20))
 (segment (start 116.84 87.14) (end 116.84 90.805) (width 0.8) (layer F.Cu) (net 20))
 (segment (start 105.41 66.04) (end 107.95 66.04) (width 0.8) (layer F.Cu) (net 2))
 (segment (start 111.125 66.04) (end 107.95 66.04) (width 0.8) (layer F.Cu) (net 2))
 (segment (start 105.41 71.12) (end 107.95 71.12) (width 0.8) (layer F.Cu) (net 4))
 (segment (start 111.125 71.12) (end 107.95 71.12) (width 0.8) (layer F.Cu) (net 4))
 (segment (start 105.41 68.58) (end 107.95 68.58) (width 0.8) (layer F.Cu) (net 3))
 (segment (start 111.125 68.58) (end 107.95 68.58) (width 0.8) (layer F.Cu) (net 3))
 (segment (start 105.41 100.076) (end 107.95 100.076) (width 0.8) (layer F.Cu) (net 6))
 (segment (start 112.141 100.076) (end 112.395 100.33) (width 0.8) (layer F.Cu) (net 6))
 (segment (start 107.95 100.076) (end 112.141 100.076) (width 0.8) (layer F.Cu) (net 6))
 (segment (start 112.395 100.33) (end 112.395 99.06) (width 0.8) (layer F.Cu) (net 6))
 (segment (start 114.545 96.91) (end 116.84 96.91) (width 0.8) (layer F.Cu) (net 6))
 (segment (start 112.395 99.06) (end 114.545 96.91) (width 0.8) (layer F.Cu) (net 6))
 (segment (start 105.41 97.536) (end 107.95 94.996) (width 0.8) (layer F.Cu) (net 7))
 (segment (start 107.95 94.996) (end 109.855 93.091) (width 0.8) (layer F.Cu) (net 7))
 (segment (start 109.855 93.091) (end 109.855 91.83) (width 0.8) (layer F.Cu) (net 7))
 (segment (start 117.475 112.395) (end 118.11 113.03) (width 0.8) (layer F.Cu) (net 10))
 (segment (start 115.57 105.73) (end 115.57 112.395) (width 0.8) (layer F.Cu) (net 10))
 (segment (start 114.22 104.38) (end 115.57 105.73) (width 0.8) (layer F.Cu) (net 10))
 (segment (start 112.42 104.38) (end 114.22 104.38) (width 0.8) (layer F.Cu) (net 10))
 (segment (start 114.445 112.395) (end 115.57 112.395) (width 0.8) (layer F.Cu) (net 10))
 (segment (start 115.57 112.395) (end 117.475 112.395) (width 0.8) (layer F.Cu) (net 10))
 (via (at 109.855 106.045) (size 1.2) (drill 0.8) (layers F.Cu B.Cu) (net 10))
 (segment (start 112.42 104.38) (end 111.52 104.38) (width 0.8) (layer F.Cu) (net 10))
 (segment (start 111.52 104.38) (end 109.855 106.045) (width 0.8) (layer F.Cu) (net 10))
 (via (at 109.855 83.82) (size 1.2) (drill 0.8) (layers F.Cu B.Cu) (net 10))
 (segment (start 109.855 82.06) (end 109.855 83.82) (width 0.8) (layer F.Cu) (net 10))
 (via (at 118.745 75.565) (size 1.2) (drill 0.8) (layers F.Cu B.Cu) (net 10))
 (segment (start 118.745 77.47) (end 118.745 75.565) (width 0.8) (layer F.Cu) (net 10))
 (segment (start 116.755 75.565) (end 116.205 76.115) (width 0.8) (layer F.Cu) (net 10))
 (segment (start 118.745 75.565) (end 116.755 75.565) (width 0.8) (layer F.Cu) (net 10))
 (segment (start 107.95 97.536) (end 109.474 97.536) (width 0.8) (layer F.Cu) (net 10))
 (segment (start 112.395 94.615) (end 112.395 91.83) (width 0.8) (layer F.Cu) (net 10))
 (segment (start 109.474 97.536) (end 112.395 94.615) (width 0.8) (layer F.Cu) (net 10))
 (segment (start 113.695 100.33) (end 116.84 100.33) (width 0.8) (layer F.Cu) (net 21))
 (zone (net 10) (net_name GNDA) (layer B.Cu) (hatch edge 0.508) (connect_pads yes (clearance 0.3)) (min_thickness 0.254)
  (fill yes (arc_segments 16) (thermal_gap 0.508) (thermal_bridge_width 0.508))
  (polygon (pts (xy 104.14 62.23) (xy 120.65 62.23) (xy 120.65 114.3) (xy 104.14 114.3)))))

